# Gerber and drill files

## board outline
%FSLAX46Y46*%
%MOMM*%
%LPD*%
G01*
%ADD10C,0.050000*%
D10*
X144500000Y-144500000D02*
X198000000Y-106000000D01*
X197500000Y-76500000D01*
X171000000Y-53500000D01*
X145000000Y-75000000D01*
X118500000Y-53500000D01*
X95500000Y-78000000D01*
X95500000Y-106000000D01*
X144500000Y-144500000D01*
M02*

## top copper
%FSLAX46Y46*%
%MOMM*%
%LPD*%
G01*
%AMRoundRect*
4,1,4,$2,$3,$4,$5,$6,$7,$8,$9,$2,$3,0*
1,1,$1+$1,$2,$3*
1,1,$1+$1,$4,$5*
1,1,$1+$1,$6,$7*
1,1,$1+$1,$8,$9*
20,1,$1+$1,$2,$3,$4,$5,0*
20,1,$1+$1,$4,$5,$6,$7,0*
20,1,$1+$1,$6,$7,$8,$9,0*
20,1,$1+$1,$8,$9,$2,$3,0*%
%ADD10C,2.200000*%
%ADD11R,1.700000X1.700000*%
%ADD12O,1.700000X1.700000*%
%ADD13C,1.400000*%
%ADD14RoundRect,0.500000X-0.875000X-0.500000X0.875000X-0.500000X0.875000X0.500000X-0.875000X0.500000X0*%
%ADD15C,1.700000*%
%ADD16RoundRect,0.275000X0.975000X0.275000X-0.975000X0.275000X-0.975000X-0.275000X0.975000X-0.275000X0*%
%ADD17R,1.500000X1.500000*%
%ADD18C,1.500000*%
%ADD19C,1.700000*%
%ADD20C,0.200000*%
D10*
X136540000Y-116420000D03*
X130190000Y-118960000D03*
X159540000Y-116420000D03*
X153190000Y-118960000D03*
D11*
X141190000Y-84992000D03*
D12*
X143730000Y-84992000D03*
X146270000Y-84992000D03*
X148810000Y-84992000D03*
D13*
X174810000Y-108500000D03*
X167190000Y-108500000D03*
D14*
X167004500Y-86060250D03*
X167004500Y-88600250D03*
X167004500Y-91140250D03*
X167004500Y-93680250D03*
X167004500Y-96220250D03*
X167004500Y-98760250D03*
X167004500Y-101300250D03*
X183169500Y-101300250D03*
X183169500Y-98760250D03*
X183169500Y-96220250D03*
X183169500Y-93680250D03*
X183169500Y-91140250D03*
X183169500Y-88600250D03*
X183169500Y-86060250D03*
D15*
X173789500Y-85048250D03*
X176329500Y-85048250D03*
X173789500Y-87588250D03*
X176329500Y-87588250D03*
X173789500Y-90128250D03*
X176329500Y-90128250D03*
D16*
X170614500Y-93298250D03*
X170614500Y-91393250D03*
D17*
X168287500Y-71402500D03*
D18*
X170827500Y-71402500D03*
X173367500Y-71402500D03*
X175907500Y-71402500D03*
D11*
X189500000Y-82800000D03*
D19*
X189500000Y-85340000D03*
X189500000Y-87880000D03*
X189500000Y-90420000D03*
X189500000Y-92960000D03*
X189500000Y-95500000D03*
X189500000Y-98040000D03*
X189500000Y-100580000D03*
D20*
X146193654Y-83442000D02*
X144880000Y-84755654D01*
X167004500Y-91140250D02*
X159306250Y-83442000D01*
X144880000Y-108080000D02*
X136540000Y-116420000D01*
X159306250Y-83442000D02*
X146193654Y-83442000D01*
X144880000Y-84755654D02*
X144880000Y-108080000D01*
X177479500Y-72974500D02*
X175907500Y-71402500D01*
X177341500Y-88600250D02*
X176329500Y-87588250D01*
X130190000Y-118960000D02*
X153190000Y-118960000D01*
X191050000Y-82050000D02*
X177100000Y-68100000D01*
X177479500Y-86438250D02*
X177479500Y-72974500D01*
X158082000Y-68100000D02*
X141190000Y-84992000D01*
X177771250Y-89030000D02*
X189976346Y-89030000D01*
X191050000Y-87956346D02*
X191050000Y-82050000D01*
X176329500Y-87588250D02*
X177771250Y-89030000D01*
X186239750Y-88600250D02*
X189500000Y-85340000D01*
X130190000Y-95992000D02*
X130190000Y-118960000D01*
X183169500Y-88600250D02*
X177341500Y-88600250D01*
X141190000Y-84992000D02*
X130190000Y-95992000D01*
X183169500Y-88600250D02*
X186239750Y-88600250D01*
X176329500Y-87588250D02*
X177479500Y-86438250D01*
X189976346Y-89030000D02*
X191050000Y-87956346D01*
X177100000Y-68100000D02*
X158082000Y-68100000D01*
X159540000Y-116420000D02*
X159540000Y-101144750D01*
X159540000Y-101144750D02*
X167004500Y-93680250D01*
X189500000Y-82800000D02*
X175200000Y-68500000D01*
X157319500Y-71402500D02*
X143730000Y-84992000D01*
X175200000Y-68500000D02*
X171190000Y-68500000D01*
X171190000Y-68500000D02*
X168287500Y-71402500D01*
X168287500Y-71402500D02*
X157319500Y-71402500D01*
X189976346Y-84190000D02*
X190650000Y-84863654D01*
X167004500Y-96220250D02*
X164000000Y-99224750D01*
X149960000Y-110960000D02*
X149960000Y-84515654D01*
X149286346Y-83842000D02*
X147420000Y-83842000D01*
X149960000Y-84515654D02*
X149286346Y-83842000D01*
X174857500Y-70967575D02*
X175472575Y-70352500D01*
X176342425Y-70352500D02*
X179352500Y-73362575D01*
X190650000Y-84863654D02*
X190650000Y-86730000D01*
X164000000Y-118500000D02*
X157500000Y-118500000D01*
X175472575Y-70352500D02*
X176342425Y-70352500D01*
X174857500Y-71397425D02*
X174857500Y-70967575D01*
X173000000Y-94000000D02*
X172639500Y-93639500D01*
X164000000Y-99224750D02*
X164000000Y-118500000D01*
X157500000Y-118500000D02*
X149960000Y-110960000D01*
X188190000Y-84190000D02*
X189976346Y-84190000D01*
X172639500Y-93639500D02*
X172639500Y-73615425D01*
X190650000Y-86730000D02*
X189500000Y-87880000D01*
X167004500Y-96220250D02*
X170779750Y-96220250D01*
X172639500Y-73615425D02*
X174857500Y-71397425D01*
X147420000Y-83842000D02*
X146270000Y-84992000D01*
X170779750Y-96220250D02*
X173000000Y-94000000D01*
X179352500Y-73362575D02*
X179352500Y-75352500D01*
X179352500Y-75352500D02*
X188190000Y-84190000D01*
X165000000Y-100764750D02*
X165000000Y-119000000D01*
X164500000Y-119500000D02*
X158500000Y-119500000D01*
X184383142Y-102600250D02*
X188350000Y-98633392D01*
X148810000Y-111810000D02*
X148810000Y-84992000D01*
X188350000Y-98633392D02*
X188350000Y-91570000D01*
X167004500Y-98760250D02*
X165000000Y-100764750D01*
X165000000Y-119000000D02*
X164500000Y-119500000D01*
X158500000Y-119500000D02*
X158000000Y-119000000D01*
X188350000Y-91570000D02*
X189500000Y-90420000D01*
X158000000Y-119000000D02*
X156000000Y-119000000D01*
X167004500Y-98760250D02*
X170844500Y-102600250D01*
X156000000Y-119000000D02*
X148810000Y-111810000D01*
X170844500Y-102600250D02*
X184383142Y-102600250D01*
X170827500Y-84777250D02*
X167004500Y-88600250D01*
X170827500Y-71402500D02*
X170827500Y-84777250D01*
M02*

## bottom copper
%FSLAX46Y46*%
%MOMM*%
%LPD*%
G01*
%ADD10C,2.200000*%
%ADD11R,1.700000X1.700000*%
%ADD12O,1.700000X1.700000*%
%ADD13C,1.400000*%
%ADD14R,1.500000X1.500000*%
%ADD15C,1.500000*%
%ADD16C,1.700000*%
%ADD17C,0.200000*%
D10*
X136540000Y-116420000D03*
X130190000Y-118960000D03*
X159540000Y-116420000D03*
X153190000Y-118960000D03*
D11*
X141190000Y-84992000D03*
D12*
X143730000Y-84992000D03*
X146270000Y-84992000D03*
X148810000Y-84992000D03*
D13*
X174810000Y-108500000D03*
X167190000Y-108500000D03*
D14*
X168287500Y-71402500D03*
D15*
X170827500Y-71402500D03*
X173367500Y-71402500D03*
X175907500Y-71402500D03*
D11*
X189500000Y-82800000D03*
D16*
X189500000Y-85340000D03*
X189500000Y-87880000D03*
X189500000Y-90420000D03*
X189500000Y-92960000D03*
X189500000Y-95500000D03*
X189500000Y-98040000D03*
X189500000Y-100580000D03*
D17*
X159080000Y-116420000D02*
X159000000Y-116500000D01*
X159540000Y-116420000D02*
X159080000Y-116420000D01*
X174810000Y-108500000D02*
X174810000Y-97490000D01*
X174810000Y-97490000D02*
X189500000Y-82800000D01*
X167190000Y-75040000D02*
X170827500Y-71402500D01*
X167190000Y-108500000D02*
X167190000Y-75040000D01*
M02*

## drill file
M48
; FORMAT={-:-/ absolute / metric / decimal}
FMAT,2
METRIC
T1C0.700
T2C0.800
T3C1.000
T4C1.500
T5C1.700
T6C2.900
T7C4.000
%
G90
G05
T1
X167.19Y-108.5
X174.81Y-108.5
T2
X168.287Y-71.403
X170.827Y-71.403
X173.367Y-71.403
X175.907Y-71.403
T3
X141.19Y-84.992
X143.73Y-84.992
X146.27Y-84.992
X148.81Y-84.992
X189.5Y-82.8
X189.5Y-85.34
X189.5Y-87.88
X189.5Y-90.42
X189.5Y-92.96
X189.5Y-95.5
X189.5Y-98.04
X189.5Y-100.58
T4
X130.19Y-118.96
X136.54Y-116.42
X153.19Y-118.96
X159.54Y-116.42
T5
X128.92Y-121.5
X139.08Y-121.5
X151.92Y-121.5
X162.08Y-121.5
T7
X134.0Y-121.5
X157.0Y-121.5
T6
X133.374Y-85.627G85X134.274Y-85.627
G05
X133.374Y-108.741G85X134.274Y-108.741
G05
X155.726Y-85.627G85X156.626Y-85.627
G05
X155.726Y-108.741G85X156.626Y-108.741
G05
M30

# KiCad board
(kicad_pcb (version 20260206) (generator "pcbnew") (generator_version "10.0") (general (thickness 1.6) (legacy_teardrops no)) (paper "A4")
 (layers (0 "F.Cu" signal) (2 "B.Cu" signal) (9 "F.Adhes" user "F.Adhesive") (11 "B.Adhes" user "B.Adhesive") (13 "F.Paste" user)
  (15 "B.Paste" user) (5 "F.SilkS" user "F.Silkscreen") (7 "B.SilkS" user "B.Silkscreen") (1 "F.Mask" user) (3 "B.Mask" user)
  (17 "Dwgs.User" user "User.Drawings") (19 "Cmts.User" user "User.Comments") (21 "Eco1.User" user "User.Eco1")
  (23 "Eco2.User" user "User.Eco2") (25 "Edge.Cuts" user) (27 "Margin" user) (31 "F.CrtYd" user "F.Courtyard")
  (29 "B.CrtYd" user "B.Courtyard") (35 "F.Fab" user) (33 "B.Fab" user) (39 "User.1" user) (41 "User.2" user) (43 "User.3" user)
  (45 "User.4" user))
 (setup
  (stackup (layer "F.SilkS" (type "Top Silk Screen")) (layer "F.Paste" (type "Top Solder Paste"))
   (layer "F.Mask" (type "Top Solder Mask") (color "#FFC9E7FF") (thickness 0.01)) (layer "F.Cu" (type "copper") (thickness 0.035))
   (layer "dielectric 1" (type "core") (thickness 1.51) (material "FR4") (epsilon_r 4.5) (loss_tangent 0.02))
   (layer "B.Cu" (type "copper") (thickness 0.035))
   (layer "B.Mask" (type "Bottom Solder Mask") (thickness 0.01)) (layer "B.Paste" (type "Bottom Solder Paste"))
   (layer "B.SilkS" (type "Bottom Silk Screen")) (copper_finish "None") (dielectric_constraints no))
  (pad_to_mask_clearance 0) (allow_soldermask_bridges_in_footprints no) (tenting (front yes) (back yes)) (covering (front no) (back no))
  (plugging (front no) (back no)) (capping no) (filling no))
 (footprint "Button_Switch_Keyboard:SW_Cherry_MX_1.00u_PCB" (layer "F.Cu") (at 136.54 116.42)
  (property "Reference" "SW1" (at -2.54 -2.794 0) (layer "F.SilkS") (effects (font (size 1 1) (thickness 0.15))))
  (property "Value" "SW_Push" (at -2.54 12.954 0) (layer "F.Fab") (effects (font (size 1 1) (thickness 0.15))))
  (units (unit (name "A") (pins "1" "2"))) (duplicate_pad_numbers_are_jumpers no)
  (pad "" np_thru_hole circle (at -7.62 5.08) (size 1.7 1.7) (drill 1.7) (layers "*.Cu" "*.Mask"))
  (pad "" np_thru_hole circle (at -2.54 5.08) (size 4 4) (drill 4) (layers "*.Cu" "*.Mask"))
  (pad "" np_thru_hole circle (at 2.54 5.08) (size 1.7 1.7) (drill 1.7) (layers "*.Cu" "*.Mask"))
  (pad "1" thru_hole circle (at 0 0) (size 2.2 2.2) (drill 1.5) (layers "*.Cu" "*.Mask") (remove_unused_layers no) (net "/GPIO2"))
  (pad "2" thru_hole circle (at -6.35 2.54) (size 2.2 2.2) (drill 1.5) (layers "*.Cu" "*.Mask") (remove_unused_layers no) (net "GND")))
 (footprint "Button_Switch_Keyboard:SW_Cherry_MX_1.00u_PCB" (layer "F.Cu") (at 159.54 116.42)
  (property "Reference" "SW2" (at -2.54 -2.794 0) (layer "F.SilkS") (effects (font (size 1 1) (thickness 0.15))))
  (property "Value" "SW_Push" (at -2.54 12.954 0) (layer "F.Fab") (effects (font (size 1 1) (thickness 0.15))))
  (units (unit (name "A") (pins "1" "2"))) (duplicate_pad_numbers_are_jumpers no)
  (pad "" np_thru_hole circle (at -7.62 5.08) (size 1.7 1.7) (drill 1.7) (layers "*.Cu" "*.Mask"))
  (pad "" np_thru_hole circle (at -2.54 5.08) (size 4 4) (drill 4) (layers "*.Cu" "*.Mask"))
  (pad "" np_thru_hole circle (at 2.54 5.08) (size 1.7 1.7) (drill 1.7) (layers "*.Cu" "*.Mask"))
  (pad "1" thru_hole circle (at 0 0) (size 2.2 2.2) (drill 1.5) (layers "*.Cu" "*.Mask") (remove_unused_layers no) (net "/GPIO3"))
  (pad "2" thru_hole circle (at -6.35 2.54) (size 2.2 2.2) (drill 1.5) (layers "*.Cu" "*.Mask") (remove_unused_layers no) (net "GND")))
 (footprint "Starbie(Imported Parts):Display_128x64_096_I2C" (layer "F.Cu") (at 145 84.992)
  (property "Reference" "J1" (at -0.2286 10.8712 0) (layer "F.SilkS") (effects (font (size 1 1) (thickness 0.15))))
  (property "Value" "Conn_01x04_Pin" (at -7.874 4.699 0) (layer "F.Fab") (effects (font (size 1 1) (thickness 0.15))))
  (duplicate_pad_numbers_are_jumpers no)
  (pad "" np_thru_hole oval (at -11.176 0.635) (size 3.8 2.9) (drill oval 3.8 2.9) (layers "*.Cu" "*.Mask"))
  (pad "" np_thru_hole oval (at -11.176 23.749) (size 3.8 2.9) (drill oval 3.8 2.9) (layers "*.Cu" "*.Mask"))
  (pad "" np_thru_hole oval (at 11.176 0.635) (size 3.8 2.9) (drill oval 3.8 2.9) (layers "*.Cu" "*.Mask"))
  (pad "" np_thru_hole oval (at 11.176 23.749) (size 3.8 2.9) (drill oval 3.8 2.9) (layers "*.Cu" "*.Mask"))
  (pad "1" thru_hole rect (at -3.81 0 90) (size 1.7 1.7) (drill 1) (layers "*.Cu" "*.Mask") (remove_unused_layers no) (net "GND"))
  (pad "2" thru_hole oval (at -1.27 0 90) (size 1.7 1.7) (drill 1) (layers "*.Cu" "*.Mask") (remove_unused_layers no) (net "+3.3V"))
  (pad "3" thru_hole oval (at 1.27 0 90) (size 1.7 1.7) (drill 1) (layers "*.Cu" "*.Mask") (remove_unused_layers no) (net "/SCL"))
  (pad "4" thru_hole oval (at 3.81 0 90) (size 1.7 1.7) (drill 1) (layers "*.Cu" "*.Mask") (remove_unused_layers no) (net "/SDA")))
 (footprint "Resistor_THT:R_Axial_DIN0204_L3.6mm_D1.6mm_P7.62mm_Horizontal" (layer "F.Cu") (at 174.81 108.5 180)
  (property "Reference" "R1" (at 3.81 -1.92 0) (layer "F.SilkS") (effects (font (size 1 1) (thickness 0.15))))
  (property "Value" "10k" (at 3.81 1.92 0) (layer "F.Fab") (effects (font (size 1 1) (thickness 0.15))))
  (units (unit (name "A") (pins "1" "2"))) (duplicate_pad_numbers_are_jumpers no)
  (pad "1" thru_hole circle (at 0 0 180) (size 1.4 1.4) (drill 0.7) (layers "*.Cu" "*.Mask") (remove_unused_layers no) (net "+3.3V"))
  (pad "2" thru_hole circle (at 7.62 0 180) (size 1.4 1.4) (drill 0.7) (layers "*.Cu" "*.Mask") (remove_unused_layers no)
   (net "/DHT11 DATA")))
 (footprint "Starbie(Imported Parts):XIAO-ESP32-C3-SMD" (layer "F.Cu") (at 166.1695 104.18025)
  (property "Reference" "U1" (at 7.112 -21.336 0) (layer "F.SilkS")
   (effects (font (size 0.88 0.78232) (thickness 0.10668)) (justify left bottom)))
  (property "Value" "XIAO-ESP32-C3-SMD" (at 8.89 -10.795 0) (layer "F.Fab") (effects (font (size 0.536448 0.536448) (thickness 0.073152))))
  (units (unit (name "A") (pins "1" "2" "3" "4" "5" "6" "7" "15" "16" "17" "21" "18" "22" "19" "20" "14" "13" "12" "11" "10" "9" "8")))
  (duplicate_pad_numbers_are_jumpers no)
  (pad "1" smd roundrect (at 0.835 -18.12) (size 2.75 2) (layers "F.Cu" "F.Mask" "F.Paste") (roundrect_rratio 0.25)
   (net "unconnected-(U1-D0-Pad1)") (solder_mask_margin 0.0508) (thermal_bridge_angle 45))
  (pad "2" smd roundrect (at 0.835 -15.58) (size 2.75 2) (layers "F.Cu" "F.Mask" "F.Paste") (roundrect_rratio 0.25) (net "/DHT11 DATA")
   (solder_mask_margin 0.0508) (thermal_bridge_angle 45))
  (pad "3" smd roundrect (at 0.835 -13.04) (size 2.75 2) (layers "F.Cu" "F.Mask" "F.Paste") (roundrect_rratio 0.25) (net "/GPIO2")
   (solder_mask_margin 0.0508) (thermal_bridge_angle 45))
  (pad "4" smd roundrect (at 0.835 -10.5) (size 2.75 2) (layers "F.Cu" "F.Mask" "F.Paste") (roundrect_rratio 0.25) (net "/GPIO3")
   (solder_mask_margin 0.0508) (thermal_bridge_angle 45))
  (pad "5" smd roundrect (at 0.835 -7.96) (size 2.75 2) (layers "F.Cu" "F.Mask" "F.Paste") (roundrect_rratio 0.25) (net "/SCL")
   (solder_mask_margin 0.0508) (thermal_bridge_angle 45))
  (pad "6" smd roundrect (at 0.835 -5.42) (size 2.75 2) (layers "F.Cu" "F.Mask" "F.Paste") (roundrect_rratio 0.25) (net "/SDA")
   (solder_mask_margin 0.0508) (thermal_bridge_angle 45))
  (pad "7" smd roundrect (at 0.835 -2.88) (size 2.75 2) (layers "F.Cu" "F.Mask" "F.Paste") (roundrect_rratio 0.25)
   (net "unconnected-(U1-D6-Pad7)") (solder_mask_margin 0.0508) (thermal_bridge_angle 45))
  (pad "8" smd roundrect (at 17 -2.88) (size 2.75 2) (layers "F.Cu" "F.Mask" "F.Paste") (roundrect_rratio 0.25)
   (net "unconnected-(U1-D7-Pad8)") (solder_mask_margin 0.0508) (thermal_bridge_angle 45))
  (pad "9" smd roundrect (at 17 -5.42) (size 2.75 2) (layers "F.Cu" "F.Mask" "F.Paste") (roundrect_rratio 0.25)
   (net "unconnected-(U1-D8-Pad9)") (solder_mask_margin 0.0508) (thermal_bridge_angle 45))
  (pad "10" smd roundrect (at 17 -7.96) (size 2.75 2) (layers "F.Cu" "F.Mask" "F.Paste") (roundrect_rratio 0.25)
   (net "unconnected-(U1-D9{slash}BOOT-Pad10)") (solder_mask_margin 0.0508) (thermal_bridge_angle 45))
  (pad "11" smd roundrect (at 17 -10.5) (size 2.75 2) (layers "F.Cu" "F.Mask" "F.Paste") (roundrect_rratio 0.25)
   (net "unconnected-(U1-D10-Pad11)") (solder_mask_margin 0.0508) (thermal_bridge_angle 45))
  (pad "12" smd roundrect (at 17 -13.04) (size 2.75 2) (layers "F.Cu" "F.Mask" "F.Paste") (roundrect_rratio 0.25) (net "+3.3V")
   (solder_mask_margin 0.0508) (thermal_bridge_angle 45))
  (pad "13" smd roundrect (at 17 -15.58) (size 2.75 2) (layers "F.Cu" "F.Mask" "F.Paste") (roundrect_rratio 0.25) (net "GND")
   (solder_mask_margin 0.0508) (thermal_bridge_angle 45))
  (pad "14" smd roundrect (at 17 -18.12) (size 2.75 2) (layers "F.Cu" "F.Mask" "F.Paste") (roundrect_rratio 0.25) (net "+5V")
   (solder_mask_margin 0.0508) (thermal_bridge_angle 45))
  (pad "15" smd circle (at 7.62 -19.132) (size 1.7 1.7) (layers "F.Cu" "F.Mask" "F.Paste") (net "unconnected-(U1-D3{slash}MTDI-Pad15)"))
  (pad "16" smd circle (at 10.16 -19.132) (size 1.7 1.7) (layers "F.Cu" "F.Mask" "F.Paste") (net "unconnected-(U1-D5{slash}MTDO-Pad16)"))
  (pad "17" smd circle (at 7.62 -16.592) (size 1.7 1.7) (layers "F.Cu" "F.Mask" "F.Paste") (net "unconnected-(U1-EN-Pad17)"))
  (pad "18" smd circle (at 10.16 -16.592) (size 1.7 1.7) (layers "F.Cu" "F.Mask" "F.Paste") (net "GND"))
  (pad "19" smd circle (at 7.62 -14.052) (size 1.7 1.7) (layers "F.Cu" "F.Mask" "F.Paste") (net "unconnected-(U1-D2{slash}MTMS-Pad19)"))
  (pad "20" smd circle (at 10.16 -14.052) (size 1.7 1.7) (layers "F.Cu" "F.Mask" "F.Paste") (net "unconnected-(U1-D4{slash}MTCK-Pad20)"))
  (pad "21" smd roundrect (at 4.445 -10.882 180) (size 2.5 1.1) (layers "F.Cu" "F.Mask" "F.Paste") (roundrect_rratio 0.25)
   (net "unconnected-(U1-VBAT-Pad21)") (thermal_bridge_angle 45))
  (pad "22" smd roundrect (at 4.445 -12.787 180) (size 2.5 1.1) (layers "F.Cu" "F.Mask" "F.Paste") (roundrect_rratio 0.25)
   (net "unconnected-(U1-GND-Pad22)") (thermal_bridge_angle 45)))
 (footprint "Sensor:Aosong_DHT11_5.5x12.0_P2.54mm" (layer "F.Cu") (at 168.2875 71.4025 90)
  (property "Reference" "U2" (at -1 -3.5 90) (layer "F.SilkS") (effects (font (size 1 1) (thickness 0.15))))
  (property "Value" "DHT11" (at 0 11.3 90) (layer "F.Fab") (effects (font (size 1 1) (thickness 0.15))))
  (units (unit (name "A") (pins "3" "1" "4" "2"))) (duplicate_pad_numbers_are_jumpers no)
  (pad "1" thru_hole rect (at 0 0 90) (size 1.5 1.5) (drill 0.8) (layers "*.Cu" "*.Mask") (remove_unused_layers no) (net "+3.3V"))
  (pad "2" thru_hole circle (at 0 2.54 90) (size 1.5 1.5) (drill 0.8) (layers "*.Cu" "*.Mask") (remove_unused_layers no) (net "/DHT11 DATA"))
  (pad "3" thru_hole circle (at 0 5.08 90) (size 1.5 1.5) (drill 0.8) (layers "*.Cu" "*.Mask") (remove_unused_layers no)
   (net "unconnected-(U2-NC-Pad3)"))
  (pad "4" thru_hole circle (at 0 7.62 90) (size 1.5 1.5) (drill 0.8) (layers "*.Cu" "*.Mask") (remove_unused_layers no) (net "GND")))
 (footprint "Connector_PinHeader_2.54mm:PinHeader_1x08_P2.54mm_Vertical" (layer "F.Cu") (at 189.5 82.8)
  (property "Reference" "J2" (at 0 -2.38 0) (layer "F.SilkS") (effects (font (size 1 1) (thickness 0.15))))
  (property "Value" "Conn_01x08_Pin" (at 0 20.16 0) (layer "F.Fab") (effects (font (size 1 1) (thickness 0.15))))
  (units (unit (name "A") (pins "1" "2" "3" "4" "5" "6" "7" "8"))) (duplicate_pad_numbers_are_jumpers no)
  (pad "1" thru_hole rect (at 0 0) (size 1.7 1.7) (drill 1) (layers "*.Cu" "*.Mask") (remove_unused_layers no) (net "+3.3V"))
  (pad "2" thru_hole circle (at 0 2.54) (size 1.7 1.7) (drill 1) (layers "*.Cu" "*.Mask") (remove_unused_layers no) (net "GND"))
  (pad "3" thru_hole circle (at 0 5.08) (size 1.7 1.7) (drill 1) (layers "*.Cu" "*.Mask") (remove_unused_layers no) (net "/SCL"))
  (pad "4" thru_hole circle (at 0 7.62) (size 1.7 1.7) (drill 1) (layers "*.Cu" "*.Mask") (remove_unused_layers no) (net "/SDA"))
  (pad "5" thru_hole circle (at 0 10.16) (size 1.7 1.7) (drill 1) (layers "*.Cu" "*.Mask") (remove_unused_layers no)
   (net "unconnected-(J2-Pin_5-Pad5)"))
  (pad "6" thru_hole circle (at 0 12.7) (size 1.7 1.7) (drill 1) (layers "*.Cu" "*.Mask") (remove_unused_layers no)
   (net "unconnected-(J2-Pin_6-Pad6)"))
  (pad "7" thru_hole circle (at 0 15.24) (size 1.7 1.7) (drill 1) (layers "*.Cu" "*.Mask") (remove_unused_layers no)
   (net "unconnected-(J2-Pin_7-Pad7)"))
  (pad "8" thru_hole circle (at 0 17.78) (size 1.7 1.7) (drill 1) (layers "*.Cu" "*.Mask") (remove_unused_layers no)
   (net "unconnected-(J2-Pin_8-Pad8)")))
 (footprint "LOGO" (layer "F.Cu") (at 146.5 99.5)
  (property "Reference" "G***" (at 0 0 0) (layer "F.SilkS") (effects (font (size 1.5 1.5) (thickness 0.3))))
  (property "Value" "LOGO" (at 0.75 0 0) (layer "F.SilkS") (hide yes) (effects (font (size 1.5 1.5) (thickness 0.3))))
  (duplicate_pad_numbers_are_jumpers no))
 (gr_poly
  (pts (xy 144.5 144.5) (xy 198 106) (xy 197.5 76.5) (xy 171 53.5) (xy 145 75) (xy 118.5 53.5) (xy 95.5 78) (xy 95.5 106))
  (stroke (width 0.05) (type solid)) (fill no) (layer "Edge.Cuts"))
 (segment (start 146.193654 83.442) (end 144.88 84.755654) (width 0.2) (layer "F.Cu") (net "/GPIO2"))
 (segment (start 167.0045 91.14025) (end 159.30625 83.442) (width 0.2) (layer "F.Cu") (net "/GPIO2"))
 (segment (start 144.88 108.08) (end 136.54 116.42) (width 0.2) (layer "F.Cu") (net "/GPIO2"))
 (segment (start 159.30625 83.442) (end 146.193654 83.442) (width 0.2) (layer "F.Cu") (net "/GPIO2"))
 (segment (start 144.88 84.755654) (end 144.88 108.08) (width 0.2) (layer "F.Cu") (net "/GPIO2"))
 (segment (start 177.4795 72.9745) (end 175.9075 71.4025) (width 0.2) (layer "F.Cu") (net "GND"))
 (segment (start 177.3415 88.60025) (end 176.3295 87.58825) (width 0.2) (layer "F.Cu") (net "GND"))
 (segment (start 130.19 118.96) (end 153.19 118.96) (width 0.2) (layer "F.Cu") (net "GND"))
 (segment (start 191.05 82.05) (end 177.1 68.1) (width 0.2) (layer "F.Cu") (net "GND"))
 (segment (start 177.4795 86.43825) (end 177.4795 72.9745) (width 0.2) (layer "F.Cu") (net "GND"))
 (segment (start 158.082 68.1) (end 141.19 84.992) (width 0.2) (layer "F.Cu") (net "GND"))
 (segment (start 177.77125 89.03) (end 189.976346 89.03) (width 0.2) (layer "F.Cu") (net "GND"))
 (segment (start 191.05 87.956346) (end 191.05 82.05) (width 0.2) (layer "F.Cu") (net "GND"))
 (segment (start 176.3295 87.58825) (end 177.77125 89.03) (width 0.2) (layer "F.Cu") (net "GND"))
 (segment (start 186.23975 88.60025) (end 189.5 85.34) (width 0.2) (layer "F.Cu") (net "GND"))
 (segment (start 130.19 95.992) (end 130.19 118.96) (width 0.2) (layer "F.Cu") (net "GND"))
 (segment (start 183.1695 88.60025) (end 177.3415 88.60025) (width 0.2) (layer "F.Cu") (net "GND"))
 (segment (start 141.19 84.992) (end 130.19 95.992) (width 0.2) (layer "F.Cu") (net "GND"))
 (segment (start 183.1695 88.60025) (end 186.23975 88.60025) (width 0.2) (layer "F.Cu") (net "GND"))
 (segment (start 176.3295 87.58825) (end 177.4795 86.43825) (width 0.2) (layer "F.Cu") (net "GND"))
 (segment (start 189.976346 89.03) (end 191.05 87.956346) (width 0.2) (layer "F.Cu") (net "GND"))
 (segment (start 177.1 68.1) (end 158.082 68.1) (width 0.2) (layer "F.Cu") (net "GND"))
 (segment (start 159.54 116.42) (end 159.54 101.14475) (width 0.2) (layer "F.Cu") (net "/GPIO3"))
 (segment (start 159.54 101.14475) (end 167.0045 93.68025) (width 0.2) (layer "F.Cu") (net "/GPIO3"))
 (segment (start 159.08 116.42) (end 159 116.5) (width 0.2) (layer "B.Cu") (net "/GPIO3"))
 (segment (start 159.54 116.42) (end 159.08 116.42) (width 0.2) (layer "B.Cu") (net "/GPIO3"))
 (segment (start 189.5 82.8) (end 175.2 68.5) (width 0.2) (layer "F.Cu") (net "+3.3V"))
 (segment (start 157.3195 71.4025) (end 143.73 84.992) (width 0.2) (layer "F.Cu") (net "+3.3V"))
 (segment (start 175.2 68.5) (end 171.19 68.5) (width 0.2) (layer "F.Cu") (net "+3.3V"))
 (segment (start 171.19 68.5) (end 168.2875 71.4025) (width 0.2) (layer "F.Cu") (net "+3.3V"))
 (segment (start 168.2875 71.4025) (end 157.3195 71.4025) (width 0.2) (layer "F.Cu") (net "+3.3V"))
 (segment (start 174.81 108.5) (end 174.81 97.49) (width 0.2) (layer "B.Cu") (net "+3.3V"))
 (segment (start 174.81 97.49) (end 189.5 82.8) (width 0.2) (layer "B.Cu") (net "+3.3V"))
 (segment (start 189.976346 84.19) (end 190.65 84.863654) (width 0.2) (layer "F.Cu") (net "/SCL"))
 (segment (start 167.0045 96.22025) (end 164 99.22475) (width 0.2) (layer "F.Cu") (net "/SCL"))
 (segment (start 149.96 110.96) (end 149.96 84.515654) (width 0.2) (layer "F.Cu") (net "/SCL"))
 (segment (start 149.286346 83.842) (end 147.42 83.842) (width 0.2) (layer "F.Cu") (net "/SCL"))
 (segment (start 149.96 84.515654) (end 149.286346 83.842) (width 0.2) (layer "F.Cu") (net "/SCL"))
 (segment (start 174.8575 70.967575) (end 175.472575 70.3525) (width 0.2) (layer "F.Cu") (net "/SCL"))
 (segment (start 176.342425 70.3525) (end 179.3525 73.362575) (width 0.2) (layer "F.Cu") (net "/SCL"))
 (segment (start 190.65 84.863654) (end 190.65 86.73) (width 0.2) (layer "F.Cu") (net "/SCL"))
 (segment (start 164 118.5) (end 157.5 118.5) (width 0.2) (layer "F.Cu") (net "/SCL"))
 (segment (start 175.472575 70.3525) (end 176.342425 70.3525) (width 0.2) (layer "F.Cu") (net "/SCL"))
 (segment (start 174.8575 71.397425) (end 174.8575 70.967575) (width 0.2) (layer "F.Cu") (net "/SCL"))
 (segment (start 173 94) (end 172.6395 93.6395) (width 0.2) (layer "F.Cu") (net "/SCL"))
 (segment (start 164 99.22475) (end 164 118.5) (width 0.2) (layer "F.Cu") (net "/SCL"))
 (segment (start 157.5 118.5) (end 149.96 110.96) (width 0.2) (layer "F.Cu") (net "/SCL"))
 (segment (start 188.19 84.19) (end 189.976346 84.19) (width 0.2) (layer "F.Cu") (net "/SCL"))
 (segment (start 172.6395 93.6395) (end 172.6395 73.615425) (width 0.2) (layer "F.Cu") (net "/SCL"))
 (segment (start 190.65 86.73) (end 189.5 87.88) (width 0.2) (layer "F.Cu") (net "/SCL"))
 (segment (start 167.0045 96.22025) (end 170.77975 96.22025) (width 0.2) (layer "F.Cu") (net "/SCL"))
 (segment (start 172.6395 73.615425) (end 174.8575 71.397425) (width 0.2) (layer "F.Cu") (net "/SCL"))
 (segment (start 147.42 83.842) (end 146.27 84.992) (width 0.2) (layer "F.Cu") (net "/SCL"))
 (segment (start 170.77975 96.22025) (end 173 94) (width 0.2) (layer "F.Cu") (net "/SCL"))
 (segment (start 179.3525 73.362575) (end 179.3525 75.3525) (width 0.2) (layer "F.Cu") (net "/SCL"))
 (segment (start 179.3525 75.3525) (end 188.19 84.19) (width 0.2) (layer "F.Cu") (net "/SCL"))
 (segment (start 165 100.76475) (end 165 119) (width 0.2) (layer "F.Cu") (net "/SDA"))
 (segment (start 164.5 119.5) (end 158.5 119.5) (width 0.2) (layer "F.Cu") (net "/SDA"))
 (segment (start 184.383142 102.60025) (end 188.35 98.633392) (width 0.2) (layer "F.Cu") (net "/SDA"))
 (segment (start 148.81 111.81) (end 148.81 84.992) (width 0.2) (layer "F.Cu") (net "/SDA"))
 (segment (start 188.35 98.633392) (end 188.35 91.57) (width 0.2) (layer "F.Cu") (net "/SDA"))
 (segment (start 167.0045 98.76025) (end 165 100.76475) (width 0.2) (layer "F.Cu") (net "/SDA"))
 (segment (start 165 119) (end 164.5 119.5) (width 0.2) (layer "F.Cu") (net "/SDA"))
 (segment (start 158.5 119.5) (end 158 119) (width 0.2) (layer "F.Cu") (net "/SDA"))
 (segment (start 188.35 91.57) (end 189.5 90.42) (width 0.2) (layer "F.Cu") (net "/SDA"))
 (segment (start 158 119) (end 156 119) (width 0.2) (layer "F.Cu") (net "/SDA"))
 (segment (start 167.0045 98.76025) (end 170.8445 102.60025) (width 0.2) (layer "F.Cu") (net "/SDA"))
 (segment (start 156 119) (end 148.81 111.81) (width 0.2) (layer "F.Cu") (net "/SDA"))
 (segment (start 170.8445 102.60025) (end 184.383142 102.60025) (width 0.2) (layer "F.Cu") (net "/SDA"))
 (segment (start 170.8275 84.77725) (end 167.0045 88.60025) (width 0.2) (layer "F.Cu") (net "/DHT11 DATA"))
 (segment (start 170.8275 71.4025) (end 170.8275 84.77725) (width 0.2) (layer "F.Cu") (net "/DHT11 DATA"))
 (segment (start 167.19 75.04) (end 170.8275 71.4025) (width 0.2) (layer "B.Cu") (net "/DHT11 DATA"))
 (segment (start 167.19 108.5) (end 167.19 75.04) (width 0.2) (layer "B.Cu") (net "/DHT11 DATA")))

